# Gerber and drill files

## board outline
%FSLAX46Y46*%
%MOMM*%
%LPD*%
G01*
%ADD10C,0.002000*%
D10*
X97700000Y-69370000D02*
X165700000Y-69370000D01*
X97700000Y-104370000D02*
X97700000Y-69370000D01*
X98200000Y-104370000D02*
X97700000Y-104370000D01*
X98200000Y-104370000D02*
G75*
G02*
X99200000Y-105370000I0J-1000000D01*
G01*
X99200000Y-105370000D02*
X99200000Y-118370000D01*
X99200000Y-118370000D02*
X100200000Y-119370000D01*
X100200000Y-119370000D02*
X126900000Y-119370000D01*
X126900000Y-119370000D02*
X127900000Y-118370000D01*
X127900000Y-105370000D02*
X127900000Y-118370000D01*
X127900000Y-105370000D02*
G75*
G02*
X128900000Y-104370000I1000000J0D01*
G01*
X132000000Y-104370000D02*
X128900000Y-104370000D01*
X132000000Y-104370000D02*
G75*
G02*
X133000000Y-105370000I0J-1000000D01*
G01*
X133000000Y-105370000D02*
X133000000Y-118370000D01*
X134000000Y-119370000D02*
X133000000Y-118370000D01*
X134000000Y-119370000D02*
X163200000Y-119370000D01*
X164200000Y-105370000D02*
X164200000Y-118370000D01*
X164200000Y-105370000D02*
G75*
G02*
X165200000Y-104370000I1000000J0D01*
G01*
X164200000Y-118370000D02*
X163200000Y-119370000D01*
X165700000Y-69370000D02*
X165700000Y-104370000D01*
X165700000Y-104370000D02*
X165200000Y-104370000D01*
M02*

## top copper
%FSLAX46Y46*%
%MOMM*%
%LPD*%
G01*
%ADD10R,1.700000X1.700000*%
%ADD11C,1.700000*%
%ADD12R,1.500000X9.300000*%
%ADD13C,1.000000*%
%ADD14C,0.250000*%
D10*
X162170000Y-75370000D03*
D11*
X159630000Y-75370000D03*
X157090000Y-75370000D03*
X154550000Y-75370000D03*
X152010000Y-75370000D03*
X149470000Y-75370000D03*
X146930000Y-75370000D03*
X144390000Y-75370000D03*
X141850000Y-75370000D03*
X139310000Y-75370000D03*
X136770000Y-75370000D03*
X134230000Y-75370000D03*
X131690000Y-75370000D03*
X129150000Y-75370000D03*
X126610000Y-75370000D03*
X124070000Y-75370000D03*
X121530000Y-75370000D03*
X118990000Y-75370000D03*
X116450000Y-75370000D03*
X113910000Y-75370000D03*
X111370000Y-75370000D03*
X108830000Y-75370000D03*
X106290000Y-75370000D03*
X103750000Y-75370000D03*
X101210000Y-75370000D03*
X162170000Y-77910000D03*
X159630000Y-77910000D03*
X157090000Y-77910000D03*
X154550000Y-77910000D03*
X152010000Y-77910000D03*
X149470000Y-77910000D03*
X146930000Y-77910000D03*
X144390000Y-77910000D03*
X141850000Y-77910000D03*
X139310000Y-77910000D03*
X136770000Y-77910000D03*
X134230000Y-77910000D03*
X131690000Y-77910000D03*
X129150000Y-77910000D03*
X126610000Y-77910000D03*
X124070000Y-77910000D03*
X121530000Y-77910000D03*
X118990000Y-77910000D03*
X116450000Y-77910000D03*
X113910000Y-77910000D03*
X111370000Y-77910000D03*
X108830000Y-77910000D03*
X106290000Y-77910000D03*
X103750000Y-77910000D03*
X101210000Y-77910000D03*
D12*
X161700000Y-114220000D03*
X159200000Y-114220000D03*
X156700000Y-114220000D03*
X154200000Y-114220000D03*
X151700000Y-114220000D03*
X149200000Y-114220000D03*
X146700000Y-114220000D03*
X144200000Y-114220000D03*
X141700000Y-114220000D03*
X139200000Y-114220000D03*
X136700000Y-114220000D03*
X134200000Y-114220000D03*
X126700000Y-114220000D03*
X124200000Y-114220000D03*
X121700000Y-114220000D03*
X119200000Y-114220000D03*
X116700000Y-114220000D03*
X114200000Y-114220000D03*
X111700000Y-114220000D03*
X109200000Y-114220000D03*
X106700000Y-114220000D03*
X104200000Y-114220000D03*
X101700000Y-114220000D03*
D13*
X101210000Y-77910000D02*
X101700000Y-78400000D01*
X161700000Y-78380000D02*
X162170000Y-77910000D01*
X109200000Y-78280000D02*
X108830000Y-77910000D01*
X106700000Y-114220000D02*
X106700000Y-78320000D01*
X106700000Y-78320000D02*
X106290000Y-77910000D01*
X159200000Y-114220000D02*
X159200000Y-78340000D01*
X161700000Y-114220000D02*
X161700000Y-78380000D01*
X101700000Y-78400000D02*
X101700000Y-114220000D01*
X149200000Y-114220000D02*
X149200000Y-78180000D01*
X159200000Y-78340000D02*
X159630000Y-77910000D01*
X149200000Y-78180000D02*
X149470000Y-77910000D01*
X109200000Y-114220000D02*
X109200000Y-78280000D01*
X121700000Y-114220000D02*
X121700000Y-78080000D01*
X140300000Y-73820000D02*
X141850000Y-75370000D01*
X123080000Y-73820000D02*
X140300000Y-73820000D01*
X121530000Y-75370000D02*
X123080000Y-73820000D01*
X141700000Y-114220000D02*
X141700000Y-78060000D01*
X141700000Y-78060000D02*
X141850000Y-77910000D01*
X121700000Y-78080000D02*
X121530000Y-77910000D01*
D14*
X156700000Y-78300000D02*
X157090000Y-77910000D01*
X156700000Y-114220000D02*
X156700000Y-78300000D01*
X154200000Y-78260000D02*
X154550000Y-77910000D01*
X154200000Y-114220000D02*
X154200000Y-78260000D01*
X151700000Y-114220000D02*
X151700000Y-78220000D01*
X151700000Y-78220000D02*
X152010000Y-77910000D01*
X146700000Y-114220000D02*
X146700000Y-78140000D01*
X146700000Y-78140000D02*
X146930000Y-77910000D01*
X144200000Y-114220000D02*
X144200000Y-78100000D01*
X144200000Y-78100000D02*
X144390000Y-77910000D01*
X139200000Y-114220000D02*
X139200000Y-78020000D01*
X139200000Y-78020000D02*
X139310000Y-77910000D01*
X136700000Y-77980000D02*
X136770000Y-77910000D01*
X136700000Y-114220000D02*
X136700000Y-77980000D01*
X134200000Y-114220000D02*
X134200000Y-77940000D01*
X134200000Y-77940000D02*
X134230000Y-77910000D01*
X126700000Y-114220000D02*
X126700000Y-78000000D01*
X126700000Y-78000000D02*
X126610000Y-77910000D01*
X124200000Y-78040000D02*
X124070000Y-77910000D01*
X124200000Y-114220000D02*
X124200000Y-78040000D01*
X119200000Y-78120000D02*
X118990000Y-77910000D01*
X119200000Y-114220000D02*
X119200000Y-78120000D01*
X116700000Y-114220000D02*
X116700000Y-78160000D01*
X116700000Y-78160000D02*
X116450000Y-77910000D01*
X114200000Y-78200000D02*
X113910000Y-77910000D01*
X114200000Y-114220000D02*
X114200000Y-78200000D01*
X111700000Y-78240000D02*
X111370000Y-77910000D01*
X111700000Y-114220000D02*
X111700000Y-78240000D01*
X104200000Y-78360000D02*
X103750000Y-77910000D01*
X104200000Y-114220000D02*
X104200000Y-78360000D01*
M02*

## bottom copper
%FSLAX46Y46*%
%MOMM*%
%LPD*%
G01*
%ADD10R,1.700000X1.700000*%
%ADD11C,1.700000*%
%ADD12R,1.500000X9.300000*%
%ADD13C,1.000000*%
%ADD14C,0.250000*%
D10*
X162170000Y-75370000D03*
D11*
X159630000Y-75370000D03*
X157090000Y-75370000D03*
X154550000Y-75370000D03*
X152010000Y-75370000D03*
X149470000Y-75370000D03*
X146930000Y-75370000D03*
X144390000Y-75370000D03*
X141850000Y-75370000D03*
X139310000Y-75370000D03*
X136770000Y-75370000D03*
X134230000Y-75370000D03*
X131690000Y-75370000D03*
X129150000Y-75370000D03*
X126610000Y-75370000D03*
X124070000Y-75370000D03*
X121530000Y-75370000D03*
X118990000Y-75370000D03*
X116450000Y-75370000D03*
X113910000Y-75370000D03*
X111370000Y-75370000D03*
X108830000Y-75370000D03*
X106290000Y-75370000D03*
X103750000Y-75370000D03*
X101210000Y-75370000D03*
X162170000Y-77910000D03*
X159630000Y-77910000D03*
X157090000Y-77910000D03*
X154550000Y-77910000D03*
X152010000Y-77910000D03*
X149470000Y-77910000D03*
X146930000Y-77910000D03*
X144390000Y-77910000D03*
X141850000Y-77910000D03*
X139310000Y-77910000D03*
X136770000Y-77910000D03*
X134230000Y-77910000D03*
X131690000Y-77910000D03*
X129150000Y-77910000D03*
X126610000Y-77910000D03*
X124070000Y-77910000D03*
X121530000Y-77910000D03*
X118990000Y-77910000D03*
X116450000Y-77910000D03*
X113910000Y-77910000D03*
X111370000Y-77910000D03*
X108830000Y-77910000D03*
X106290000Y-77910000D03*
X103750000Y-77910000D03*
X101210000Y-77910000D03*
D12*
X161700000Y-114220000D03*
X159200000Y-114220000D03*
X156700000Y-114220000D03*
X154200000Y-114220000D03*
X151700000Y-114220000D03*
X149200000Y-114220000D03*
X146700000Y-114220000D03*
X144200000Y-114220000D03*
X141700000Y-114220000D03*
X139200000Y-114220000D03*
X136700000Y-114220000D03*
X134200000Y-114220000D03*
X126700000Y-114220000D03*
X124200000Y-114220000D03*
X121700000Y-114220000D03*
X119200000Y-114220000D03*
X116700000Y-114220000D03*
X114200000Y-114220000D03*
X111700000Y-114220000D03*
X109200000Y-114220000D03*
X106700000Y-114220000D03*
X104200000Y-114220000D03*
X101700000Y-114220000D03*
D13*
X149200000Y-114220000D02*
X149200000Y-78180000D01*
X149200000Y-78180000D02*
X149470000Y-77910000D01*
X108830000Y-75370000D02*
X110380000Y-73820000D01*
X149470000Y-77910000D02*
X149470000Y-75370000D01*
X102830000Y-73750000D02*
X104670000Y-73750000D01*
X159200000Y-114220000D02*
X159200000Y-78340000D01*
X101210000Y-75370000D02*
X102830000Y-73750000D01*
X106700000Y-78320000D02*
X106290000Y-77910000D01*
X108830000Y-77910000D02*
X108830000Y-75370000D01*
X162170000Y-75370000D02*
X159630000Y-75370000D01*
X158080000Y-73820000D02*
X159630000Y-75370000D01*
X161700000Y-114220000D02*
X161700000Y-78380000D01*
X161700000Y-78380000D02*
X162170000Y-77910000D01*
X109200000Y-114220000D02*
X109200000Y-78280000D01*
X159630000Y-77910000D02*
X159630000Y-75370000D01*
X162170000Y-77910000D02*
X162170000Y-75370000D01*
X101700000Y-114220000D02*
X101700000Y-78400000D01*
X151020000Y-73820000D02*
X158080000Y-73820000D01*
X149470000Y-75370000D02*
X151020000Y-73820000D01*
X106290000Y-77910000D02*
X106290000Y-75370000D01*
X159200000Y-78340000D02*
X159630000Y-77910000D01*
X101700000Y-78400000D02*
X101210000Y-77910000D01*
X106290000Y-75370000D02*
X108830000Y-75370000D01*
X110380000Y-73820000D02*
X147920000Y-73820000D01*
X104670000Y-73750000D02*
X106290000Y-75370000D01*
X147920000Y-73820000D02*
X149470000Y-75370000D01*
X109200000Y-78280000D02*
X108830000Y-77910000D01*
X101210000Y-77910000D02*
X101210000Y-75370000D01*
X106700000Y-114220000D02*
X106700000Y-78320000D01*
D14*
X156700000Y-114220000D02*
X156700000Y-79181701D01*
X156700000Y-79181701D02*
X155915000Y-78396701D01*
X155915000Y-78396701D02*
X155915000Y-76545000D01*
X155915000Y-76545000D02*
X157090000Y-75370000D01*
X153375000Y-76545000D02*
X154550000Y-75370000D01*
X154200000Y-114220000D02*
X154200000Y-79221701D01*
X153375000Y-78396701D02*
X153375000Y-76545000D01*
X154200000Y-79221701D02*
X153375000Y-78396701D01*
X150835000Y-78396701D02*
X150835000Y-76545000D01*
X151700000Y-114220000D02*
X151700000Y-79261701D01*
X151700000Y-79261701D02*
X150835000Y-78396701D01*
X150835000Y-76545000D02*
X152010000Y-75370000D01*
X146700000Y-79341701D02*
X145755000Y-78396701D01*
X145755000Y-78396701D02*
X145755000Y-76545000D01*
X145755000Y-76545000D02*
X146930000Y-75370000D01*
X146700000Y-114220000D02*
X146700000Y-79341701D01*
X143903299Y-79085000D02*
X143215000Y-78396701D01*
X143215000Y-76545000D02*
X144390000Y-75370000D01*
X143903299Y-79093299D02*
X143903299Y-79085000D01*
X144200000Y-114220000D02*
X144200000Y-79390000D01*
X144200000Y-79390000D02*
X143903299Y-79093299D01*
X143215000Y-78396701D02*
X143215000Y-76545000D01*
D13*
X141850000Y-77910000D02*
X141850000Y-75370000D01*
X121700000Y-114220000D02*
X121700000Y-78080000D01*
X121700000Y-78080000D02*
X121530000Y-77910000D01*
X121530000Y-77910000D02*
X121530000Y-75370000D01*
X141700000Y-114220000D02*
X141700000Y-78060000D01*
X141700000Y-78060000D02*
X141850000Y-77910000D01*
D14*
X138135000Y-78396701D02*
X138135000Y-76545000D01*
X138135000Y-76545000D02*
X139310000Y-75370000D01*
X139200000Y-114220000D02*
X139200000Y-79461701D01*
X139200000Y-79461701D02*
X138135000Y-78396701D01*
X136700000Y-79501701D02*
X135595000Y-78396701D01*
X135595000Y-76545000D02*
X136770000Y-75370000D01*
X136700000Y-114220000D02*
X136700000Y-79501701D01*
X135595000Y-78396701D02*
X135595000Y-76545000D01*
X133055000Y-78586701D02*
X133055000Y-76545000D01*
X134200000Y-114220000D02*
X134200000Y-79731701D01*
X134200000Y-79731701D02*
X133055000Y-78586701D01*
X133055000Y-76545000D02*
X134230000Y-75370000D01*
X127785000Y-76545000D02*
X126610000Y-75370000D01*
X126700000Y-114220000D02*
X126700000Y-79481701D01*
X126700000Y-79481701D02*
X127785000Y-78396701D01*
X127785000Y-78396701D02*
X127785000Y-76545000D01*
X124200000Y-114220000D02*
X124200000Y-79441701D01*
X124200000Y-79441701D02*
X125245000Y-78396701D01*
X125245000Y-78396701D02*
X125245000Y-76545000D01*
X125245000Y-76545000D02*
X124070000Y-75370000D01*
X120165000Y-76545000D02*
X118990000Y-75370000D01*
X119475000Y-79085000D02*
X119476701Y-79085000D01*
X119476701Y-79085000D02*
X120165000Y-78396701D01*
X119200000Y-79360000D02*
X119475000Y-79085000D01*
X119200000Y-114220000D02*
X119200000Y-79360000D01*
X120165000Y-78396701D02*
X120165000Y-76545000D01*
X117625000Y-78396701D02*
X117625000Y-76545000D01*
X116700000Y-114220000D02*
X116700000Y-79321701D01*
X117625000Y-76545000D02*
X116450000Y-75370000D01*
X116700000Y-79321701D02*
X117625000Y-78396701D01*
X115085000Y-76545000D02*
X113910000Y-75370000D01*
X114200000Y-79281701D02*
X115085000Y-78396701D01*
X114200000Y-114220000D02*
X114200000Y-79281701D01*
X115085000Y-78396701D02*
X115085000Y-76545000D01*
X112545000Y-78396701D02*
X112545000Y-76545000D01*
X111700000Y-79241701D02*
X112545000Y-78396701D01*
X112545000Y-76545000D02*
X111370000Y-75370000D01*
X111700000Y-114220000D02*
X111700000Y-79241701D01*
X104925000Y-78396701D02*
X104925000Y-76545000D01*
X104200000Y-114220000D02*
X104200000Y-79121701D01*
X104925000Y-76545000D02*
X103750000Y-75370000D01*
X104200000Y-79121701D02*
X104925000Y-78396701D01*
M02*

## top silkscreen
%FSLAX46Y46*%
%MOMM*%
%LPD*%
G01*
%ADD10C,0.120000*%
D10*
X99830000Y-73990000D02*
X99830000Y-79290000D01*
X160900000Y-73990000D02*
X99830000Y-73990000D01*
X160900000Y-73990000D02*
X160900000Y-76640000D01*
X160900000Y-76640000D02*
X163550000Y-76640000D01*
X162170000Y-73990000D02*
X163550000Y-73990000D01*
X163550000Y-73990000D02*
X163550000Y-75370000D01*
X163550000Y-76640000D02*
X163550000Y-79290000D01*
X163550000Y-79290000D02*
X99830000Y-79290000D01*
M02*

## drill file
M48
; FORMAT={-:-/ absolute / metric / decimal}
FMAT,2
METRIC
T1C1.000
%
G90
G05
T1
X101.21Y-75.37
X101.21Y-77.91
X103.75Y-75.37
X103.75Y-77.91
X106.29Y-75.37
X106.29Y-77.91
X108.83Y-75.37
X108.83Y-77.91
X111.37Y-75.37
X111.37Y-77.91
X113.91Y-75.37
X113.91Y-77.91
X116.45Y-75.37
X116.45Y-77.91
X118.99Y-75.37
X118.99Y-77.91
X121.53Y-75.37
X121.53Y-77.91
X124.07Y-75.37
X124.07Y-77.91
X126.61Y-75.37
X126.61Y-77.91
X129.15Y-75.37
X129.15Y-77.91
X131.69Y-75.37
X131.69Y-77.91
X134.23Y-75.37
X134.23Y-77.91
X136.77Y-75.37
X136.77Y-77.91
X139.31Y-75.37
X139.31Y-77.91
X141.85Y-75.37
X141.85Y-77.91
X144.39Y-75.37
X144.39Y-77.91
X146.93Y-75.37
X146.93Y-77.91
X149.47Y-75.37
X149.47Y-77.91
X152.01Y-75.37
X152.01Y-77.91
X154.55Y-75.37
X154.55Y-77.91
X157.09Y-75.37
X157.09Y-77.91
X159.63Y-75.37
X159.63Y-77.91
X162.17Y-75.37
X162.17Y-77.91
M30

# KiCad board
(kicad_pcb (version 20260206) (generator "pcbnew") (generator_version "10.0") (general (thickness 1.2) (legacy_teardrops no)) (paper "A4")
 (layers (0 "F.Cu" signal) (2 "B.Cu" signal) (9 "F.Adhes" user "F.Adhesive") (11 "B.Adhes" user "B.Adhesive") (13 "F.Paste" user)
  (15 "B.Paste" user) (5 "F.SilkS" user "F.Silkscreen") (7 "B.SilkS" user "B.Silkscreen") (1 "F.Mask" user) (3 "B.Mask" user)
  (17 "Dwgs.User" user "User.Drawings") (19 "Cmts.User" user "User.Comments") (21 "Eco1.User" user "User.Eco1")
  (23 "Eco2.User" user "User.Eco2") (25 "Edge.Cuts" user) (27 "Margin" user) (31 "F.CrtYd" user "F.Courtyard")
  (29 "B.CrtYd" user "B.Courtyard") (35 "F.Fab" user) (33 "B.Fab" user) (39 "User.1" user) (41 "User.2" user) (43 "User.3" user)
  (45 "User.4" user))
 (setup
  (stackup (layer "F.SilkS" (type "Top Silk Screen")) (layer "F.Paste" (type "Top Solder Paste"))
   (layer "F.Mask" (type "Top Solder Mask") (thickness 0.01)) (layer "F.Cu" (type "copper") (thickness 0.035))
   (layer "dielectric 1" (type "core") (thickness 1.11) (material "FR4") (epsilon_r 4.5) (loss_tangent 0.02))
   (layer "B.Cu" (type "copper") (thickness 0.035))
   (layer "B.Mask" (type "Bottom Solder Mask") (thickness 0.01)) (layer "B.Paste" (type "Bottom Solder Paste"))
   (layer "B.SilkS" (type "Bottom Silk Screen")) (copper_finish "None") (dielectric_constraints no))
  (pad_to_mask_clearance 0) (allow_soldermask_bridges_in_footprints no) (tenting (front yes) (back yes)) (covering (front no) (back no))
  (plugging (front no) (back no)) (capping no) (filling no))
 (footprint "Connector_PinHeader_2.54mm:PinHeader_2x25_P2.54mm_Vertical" (layer "F.Cu") (at 162.17 75.37 -90)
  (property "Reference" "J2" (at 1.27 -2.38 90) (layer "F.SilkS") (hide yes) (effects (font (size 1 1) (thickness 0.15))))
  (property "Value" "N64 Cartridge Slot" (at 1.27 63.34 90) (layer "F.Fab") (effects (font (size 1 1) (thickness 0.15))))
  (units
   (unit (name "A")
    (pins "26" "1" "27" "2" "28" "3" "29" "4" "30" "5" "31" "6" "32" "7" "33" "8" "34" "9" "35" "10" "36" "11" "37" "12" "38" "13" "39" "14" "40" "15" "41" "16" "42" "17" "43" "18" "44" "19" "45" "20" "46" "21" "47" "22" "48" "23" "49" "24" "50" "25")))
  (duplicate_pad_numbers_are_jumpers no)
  (fp_line (start -1.38 62.34) (end 3.92 62.34) (stroke (width 0.12) (type solid)) (layer "F.SilkS"))
  (fp_line (start -1.38 1.27) (end -1.38 62.34) (stroke (width 0.12) (type solid)) (layer "F.SilkS"))
  (fp_line (start -1.38 1.27) (end 1.27 1.27) (stroke (width 0.12) (type solid)) (layer "F.SilkS"))
  (fp_line (start 1.27 1.27) (end 1.27 -1.38) (stroke (width 0.12) (type solid)) (layer "F.SilkS"))
  (fp_line (start -1.38 0) (end -1.38 -1.38) (stroke (width 0.12) (type solid)) (layer "F.SilkS"))
  (fp_line (start -1.38 -1.38) (end 0 -1.38) (stroke (width 0.12) (type solid)) (layer "F.SilkS"))
  (fp_line (start 1.27 -1.38) (end 3.92 -1.38) (stroke (width 0.12) (type solid)) (layer "F.SilkS"))
  (fp_line (start 3.92 -1.38) (end 3.92 62.34) (stroke (width 0.12) (type solid)) (layer "F.SilkS"))
  (pad "1" thru_hole rect (at 0 0 270) (size 1.7 1.7) (drill 1) (layers "*.Cu" "*.Mask") (remove_unused_layers no) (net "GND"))
  (pad "2" thru_hole circle (at 0 2.54 270) (size 1.7 1.7) (drill 1) (layers "*.Cu" "*.Mask") (remove_unused_layers no) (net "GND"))
  (pad "3" thru_hole circle (at 0 5.08 270) (size 1.7 1.7) (drill 1) (layers "*.Cu" "*.Mask") (remove_unused_layers no) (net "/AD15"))
  (pad "4" thru_hole circle (at 0 7.62 270) (size 1.7 1.7) (drill 1) (layers "*.Cu" "*.Mask") (remove_unused_layers no) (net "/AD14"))
  (pad "5" thru_hole circle (at 0 10.16 270) (size 1.7 1.7) (drill 1) (layers "*.Cu" "*.Mask") (remove_unused_layers no) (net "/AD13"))
  (pad "6" thru_hole circle (at 0 12.7 270) (size 1.7 1.7) (drill 1) (layers "*.Cu" "*.Mask") (remove_unused_layers no) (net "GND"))
  (pad "7" thru_hole circle (at 0 15.24 270) (size 1.7 1.7) (drill 1) (layers "*.Cu" "*.Mask") (remove_unused_layers no) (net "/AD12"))
  (pad "8" thru_hole circle (at 0 17.78 270) (size 1.7 1.7) (drill 1) (layers "*.Cu" "*.Mask") (remove_unused_layers no) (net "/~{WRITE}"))
  (pad "9" thru_hole circle (at 0 20.32 270) (size 1.7 1.7) (drill 1) (layers "*.Cu" "*.Mask") (remove_unused_layers no) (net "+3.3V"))
  (pad "10" thru_hole circle (at 0 22.86 270) (size 1.7 1.7) (drill 1) (layers "*.Cu" "*.Mask") (remove_unused_layers no) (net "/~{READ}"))
  (pad "11" thru_hole circle (at 0 25.4 270) (size 1.7 1.7) (drill 1) (layers "*.Cu" "*.Mask") (remove_unused_layers no) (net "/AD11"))
  (pad "12" thru_hole circle (at 0 27.94 270) (size 1.7 1.7) (drill 1) (layers "*.Cu" "*.Mask") (remove_unused_layers no) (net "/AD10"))
  (pad "13" thru_hole circle (at 0 30.48 270) (size 1.7 1.7) (drill 1) (layers "*.Cu" "*.Mask") (remove_unused_layers no)
   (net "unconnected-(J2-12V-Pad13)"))
  (pad "14" thru_hole circle (at 0 33.02 270) (size 1.7 1.7) (drill 1) (layers "*.Cu" "*.Mask") (remove_unused_layers no)
   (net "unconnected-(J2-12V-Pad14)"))
  (pad "15" thru_hole circle (at 0 35.56 270) (size 1.7 1.7) (drill 1) (layers "*.Cu" "*.Mask") (remove_unused_layers no) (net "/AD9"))
  (pad "16" thru_hole circle (at 0 38.1 270) (size 1.7 1.7) (drill 1) (layers "*.Cu" "*.Mask") (remove_unused_layers no) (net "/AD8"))
  (pad "17" thru_hole circle (at 0 40.64 270) (size 1.7 1.7) (drill 1) (layers "*.Cu" "*.Mask") (remove_unused_layers no) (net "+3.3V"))
  (pad "18" thru_hole circle (at 0 43.18 270) (size 1.7 1.7) (drill 1) (layers "*.Cu" "*.Mask") (remove_unused_layers no) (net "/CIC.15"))
  (pad "19" thru_hole circle (at 0 45.72 270) (size 1.7 1.7) (drill 1) (layers "*.Cu" "*.Mask") (remove_unused_layers no) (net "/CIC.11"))
  (pad "20" thru_hole circle (at 0 48.26 270) (size 1.7 1.7) (drill 1) (layers "*.Cu" "*.Mask") (remove_unused_layers no)
   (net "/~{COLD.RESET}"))
  (pad "21" thru_hole circle (at 0 50.8 270) (size 1.7 1.7) (drill 1) (layers "*.Cu" "*.Mask") (remove_unused_layers no) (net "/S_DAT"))
  (pad "22" thru_hole circle (at 0 53.34 270) (size 1.7 1.7) (drill 1) (layers "*.Cu" "*.Mask") (remove_unused_layers no) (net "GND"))
  (pad "23" thru_hole circle (at 0 55.88 270) (size 1.7 1.7) (drill 1) (layers "*.Cu" "*.Mask") (remove_unused_layers no) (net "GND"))
  (pad "24" thru_hole circle (at 0 58.42 270) (size 1.7 1.7) (drill 1) (layers "*.Cu" "*.Mask") (remove_unused_layers no) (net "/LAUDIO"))
  (pad "25" thru_hole circle (at 0 60.96 270) (size 1.7 1.7) (drill 1) (layers "*.Cu" "*.Mask") (remove_unused_layers no) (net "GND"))
  (pad "26" thru_hole circle (at 2.54 0 270) (size 1.7 1.7) (drill 1) (layers "*.Cu" "*.Mask") (remove_unused_layers no) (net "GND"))
  (pad "27" thru_hole circle (at 2.54 2.54 270) (size 1.7 1.7) (drill 1) (layers "*.Cu" "*.Mask") (remove_unused_layers no) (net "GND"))
  (pad "28" thru_hole circle (at 2.54 5.08 270) (size 1.7 1.7) (drill 1) (layers "*.Cu" "*.Mask") (remove_unused_layers no) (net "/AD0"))
  (pad "29" thru_hole circle (at 2.54 7.62 270) (size 1.7 1.7) (drill 1) (layers "*.Cu" "*.Mask") (remove_unused_layers no) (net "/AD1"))
  (pad "30" thru_hole circle (at 2.54 10.16 270) (size 1.7 1.7) (drill 1) (layers "*.Cu" "*.Mask") (remove_unused_layers no) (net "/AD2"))
  (pad "31" thru_hole circle (at 2.54 12.7 270) (size 1.7 1.7) (drill 1) (layers "*.Cu" "*.Mask") (remove_unused_layers no) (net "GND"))
  (pad "32" thru_hole circle (at 2.54 15.24 270) (size 1.7 1.7) (drill 1) (layers "*.Cu" "*.Mask") (remove_unused_layers no) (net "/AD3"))
  (pad "33" thru_hole circle (at 2.54 17.78 270) (size 1.7 1.7) (drill 1) (layers "*.Cu" "*.Mask") (remove_unused_layers no) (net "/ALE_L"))
  (pad "34" thru_hole circle (at 2.54 20.32 270) (size 1.7 1.7) (drill 1) (layers "*.Cu" "*.Mask") (remove_unused_layers no) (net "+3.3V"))
  (pad "35" thru_hole circle (at 2.54 22.86 270) (size 1.7 1.7) (drill 1) (layers "*.Cu" "*.Mask") (remove_unused_layers no) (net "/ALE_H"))
  (pad "36" thru_hole circle (at 2.54 25.4 270) (size 1.7 1.7) (drill 1) (layers "*.Cu" "*.Mask") (remove_unused_layers no) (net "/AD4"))
  (pad "37" thru_hole circle (at 2.54 27.94 270) (size 1.7 1.7) (drill 1) (layers "*.Cu" "*.Mask") (remove_unused_layers no) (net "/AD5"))
  (pad "38" thru_hole circle (at 2.54 30.48 270) (size 1.7 1.7) (drill 1) (layers "*.Cu" "*.Mask") (remove_unused_layers no)
   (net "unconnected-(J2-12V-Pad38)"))
  (pad "39" thru_hole circle (at 2.54 33.02 270) (size 1.7 1.7) (drill 1) (layers "*.Cu" "*.Mask") (remove_unused_layers no)
   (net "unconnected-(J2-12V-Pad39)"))
  (pad "40" thru_hole circle (at 2.54 35.56 270) (size 1.7 1.7) (drill 1) (layers "*.Cu" "*.Mask") (remove_unused_layers no) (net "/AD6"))
  (pad "41" thru_hole circle (at 2.54 38.1 270) (size 1.7 1.7) (drill 1) (layers "*.Cu" "*.Mask") (remove_unused_layers no) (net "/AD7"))
  (pad "42" thru_hole circle (at 2.54 40.64 270) (size 1.7 1.7) (drill 1) (layers "*.Cu" "*.Mask") (remove_unused_layers no) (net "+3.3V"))
  (pad "43" thru_hole circle (at 2.54 43.18 270) (size 1.7 1.7) (drill 1) (layers "*.Cu" "*.Mask") (remove_unused_layers no) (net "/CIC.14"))
  (pad "44" thru_hole circle (at 2.54 45.72 270) (size 1.7 1.7) (drill 1) (layers "*.Cu" "*.Mask") (remove_unused_layers no)
   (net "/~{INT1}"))
  (pad "45" thru_hole circle (at 2.54 48.26 270) (size 1.7 1.7) (drill 1) (layers "*.Cu" "*.Mask") (remove_unused_layers no) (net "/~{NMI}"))
  (pad "46" thru_hole circle (at 2.54 50.8 270) (size 1.7 1.7) (drill 1) (layers "*.Cu" "*.Mask") (remove_unused_layers no)
   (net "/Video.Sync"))
  (pad "47" thru_hole circle (at 2.54 53.34 270) (size 1.7 1.7) (drill 1) (layers "*.Cu" "*.Mask") (remove_unused_layers no) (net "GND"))
  (pad "48" thru_hole circle (at 2.54 55.88 270) (size 1.7 1.7) (drill 1) (layers "*.Cu" "*.Mask") (remove_unused_layers no) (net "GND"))
  (pad "49" thru_hole circle (at 2.54 58.42 270) (size 1.7 1.7) (drill 1) (layers "*.Cu" "*.Mask") (remove_unused_layers no) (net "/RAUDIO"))
  (pad "50" thru_hole circle (at 2.54 60.96 270) (size 1.7 1.7) (drill 1) (layers "*.Cu" "*.Mask") (remove_unused_layers no) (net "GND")))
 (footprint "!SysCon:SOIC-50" (layer "B.Cu") (at 131.7 114.22)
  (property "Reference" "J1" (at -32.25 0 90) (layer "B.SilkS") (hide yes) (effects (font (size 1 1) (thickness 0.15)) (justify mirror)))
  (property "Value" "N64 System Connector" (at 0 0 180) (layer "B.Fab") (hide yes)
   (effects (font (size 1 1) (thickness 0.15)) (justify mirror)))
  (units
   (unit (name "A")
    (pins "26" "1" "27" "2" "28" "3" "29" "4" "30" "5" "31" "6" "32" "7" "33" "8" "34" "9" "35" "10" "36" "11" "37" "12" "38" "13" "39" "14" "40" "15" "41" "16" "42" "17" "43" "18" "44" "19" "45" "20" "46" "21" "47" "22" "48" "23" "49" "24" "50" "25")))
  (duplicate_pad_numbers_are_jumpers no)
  (pad "1" smd rect (at 30 0) (size 1.5 9.3) (layers "B.Cu" "B.Mask" "B.Paste") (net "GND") (thermal_bridge_angle 45))
  (pad "2" smd rect (at 27.5 0) (size 1.5 9.3) (layers "B.Cu" "B.Mask" "B.Paste") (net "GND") (thermal_bridge_angle 45))
  (pad "3" smd rect (at 25 0) (size 1.5 9.3) (layers "B.Cu" "B.Mask" "B.Paste") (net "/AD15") (thermal_bridge_angle 45))
  (pad "4" smd rect (at 22.5 0) (size 1.5 9.3) (layers "B.Cu" "B.Mask" "B.Paste") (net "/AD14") (thermal_bridge_angle 45))
  (pad "5" smd rect (at 20 0) (size 1.5 9.3) (layers "B.Cu" "B.Mask" "B.Paste") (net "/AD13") (thermal_bridge_angle 45))
  (pad "6" smd rect (at 17.5 0) (size 1.5 9.3) (layers "B.Cu" "B.Mask" "B.Paste") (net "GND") (thermal_bridge_angle 45))
  (pad "7" smd rect (at 15 0) (size 1.5 9.3) (layers "B.Cu" "B.Mask" "B.Paste") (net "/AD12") (thermal_bridge_angle 45))
  (pad "8" smd rect (at 12.5 0) (size 1.5 9.3) (layers "B.Cu" "B.Mask" "B.Paste") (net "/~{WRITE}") (thermal_bridge_angle 45))
  (pad "9" smd rect (at 10 0) (size 1.5 9.3) (layers "B.Cu" "B.Mask" "B.Paste") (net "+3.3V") (thermal_bridge_angle 45))
  (pad "10" smd rect (at 7.5 0) (size 1.5 9.3) (layers "B.Cu" "B.Mask" "B.Paste") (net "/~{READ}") (thermal_bridge_angle 45))
  (pad "11" smd rect (at 5 0) (size 1.5 9.3) (layers "B.Cu" "B.Mask" "B.Paste") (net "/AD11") (thermal_bridge_angle 45))
  (pad "12" smd rect (at 2.5 0) (size 1.5 9.3) (layers "B.Cu" "B.Mask" "B.Paste") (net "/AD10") (thermal_bridge_angle 45))
  (pad "15" smd rect (at -5 0) (size 1.5 9.3) (layers "B.Cu" "B.Mask" "B.Paste") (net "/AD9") (thermal_bridge_angle 45))
  (pad "16" smd rect (at -7.5 0) (size 1.5 9.3) (layers "B.Cu" "B.Mask" "B.Paste") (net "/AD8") (thermal_bridge_angle 45))
  (pad "17" smd rect (at -10 0) (size 1.5 9.3) (layers "B.Cu" "B.Mask" "B.Paste") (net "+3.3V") (thermal_bridge_angle 45))
  (pad "18" smd rect (at -12.5 0) (size 1.5 9.3) (layers "B.Cu" "B.Mask" "B.Paste") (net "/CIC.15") (thermal_bridge_angle 45))
  (pad "19" smd rect (at -15 0) (size 1.5 9.3) (layers "B.Cu" "B.Mask" "B.Paste") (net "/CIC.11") (thermal_bridge_angle 45))
  (pad "20" smd rect (at -17.5 0) (size 1.5 9.3) (layers "B.Cu" "B.Mask" "B.Paste") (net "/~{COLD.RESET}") (thermal_bridge_angle 45))
  (pad "21" smd rect (at -20 0) (size 1.5 9.3) (layers "B.Cu" "B.Mask" "B.Paste") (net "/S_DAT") (thermal_bridge_angle 45))
  (pad "22" smd rect (at -22.5 0) (size 1.5 9.3) (layers "B.Cu" "B.Mask" "B.Paste") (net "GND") (thermal_bridge_angle 45))
  (pad "23" smd rect (at -25 0) (size 1.5 9.3) (layers "B.Cu" "B.Mask" "B.Paste") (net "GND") (thermal_bridge_angle 45))
  (pad "24" smd rect (at -27.5 0) (size 1.5 9.3) (layers "B.Cu" "B.Mask" "B.Paste") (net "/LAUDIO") (thermal_bridge_angle 45))
  (pad "25" smd rect (at -30 0) (size 1.5 9.3) (layers "B.Cu" "B.Mask" "B.Paste") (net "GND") (thermal_bridge_angle 45))
  (pad "26" smd rect (at 30 0) (size 1.5 9.3) (layers "F.Cu" "F.Mask") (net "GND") (thermal_bridge_angle 45))
  (pad "27" smd rect (at 27.5 0) (size 1.5 9.3) (layers "F.Cu" "F.Mask") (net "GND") (thermal_bridge_angle 45))
  (pad "28" smd rect (at 25 0) (size 1.5 9.3) (layers "F.Cu" "F.Mask") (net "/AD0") (thermal_bridge_angle 45))
  (pad "29" smd rect (at 22.5 0) (size 1.5 9.3) (layers "F.Cu" "F.Mask") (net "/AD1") (thermal_bridge_angle 45))
  (pad "30" smd rect (at 20 0) (size 1.5 9.3) (layers "F.Cu" "F.Mask") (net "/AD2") (thermal_bridge_angle 45))
  (pad "31" smd rect (at 17.5 0) (size 1.5 9.3) (layers "F.Cu" "F.Mask") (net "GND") (thermal_bridge_angle 45))
  (pad "32" smd rect (at 15 0) (size 1.5 9.3) (layers "F.Cu" "F.Mask") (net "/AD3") (thermal_bridge_angle 45))
  (pad "33" smd rect (at 12.5 0) (size 1.5 9.3) (layers "F.Cu" "F.Mask") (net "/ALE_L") (thermal_bridge_angle 45))
  (pad "34" smd rect (at 10 0) (size 1.5 9.3) (layers "F.Cu" "F.Mask") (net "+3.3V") (thermal_bridge_angle 45))
  (pad "35" smd rect (at 7.5 0) (size 1.5 9.3) (layers "F.Cu" "F.Mask") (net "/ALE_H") (thermal_bridge_angle 45))
  (pad "36" smd rect (at 5 0) (size 1.5 9.3) (layers "F.Cu" "F.Mask") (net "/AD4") (thermal_bridge_angle 45))
  (pad "37" smd rect (at 2.5 0) (size 1.5 9.3) (layers "F.Cu" "F.Mask") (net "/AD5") (thermal_bridge_angle 45))
  (pad "40" smd rect (at -5 0) (size 1.5 9.3) (layers "F.Cu" "F.Mask") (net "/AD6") (thermal_bridge_angle 45))
  (pad "41" smd rect (at -7.5 0) (size 1.5 9.3) (layers "F.Cu" "F.Mask") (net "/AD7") (thermal_bridge_angle 45))
  (pad "42" smd rect (at -10 0) (size 1.5 9.3) (layers "F.Cu" "F.Mask") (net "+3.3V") (thermal_bridge_angle 45))
  (pad "43" smd rect (at -12.5 0) (size 1.5 9.3) (layers "F.Cu" "F.Mask") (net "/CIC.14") (thermal_bridge_angle 45))
  (pad "44" smd rect (at -15 0) (size 1.5 9.3) (layers "F.Cu" "F.Mask") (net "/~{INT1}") (thermal_bridge_angle 45))
  (pad "45" smd rect (at -17.5 0) (size 1.5 9.3) (layers "F.Cu" "F.Mask") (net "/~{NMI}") (thermal_bridge_angle 45))
  (pad "46" smd rect (at -20 0) (size 1.5 9.3) (layers "F.Cu" "F.Mask") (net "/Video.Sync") (thermal_bridge_angle 45))
  (pad "47" smd rect (at -22.5 0) (size 1.5 9.3) (layers "F.Cu" "F.Mask") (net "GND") (thermal_bridge_angle 45))
  (pad "48" smd rect (at -25 0) (size 1.5 9.3) (layers "F.Cu" "F.Mask") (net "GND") (thermal_bridge_angle 45))
  (pad "49" smd rect (at -27.5 0) (size 1.5 9.3) (layers "F.Cu" "F.Mask") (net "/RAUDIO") (thermal_bridge_angle 45))
  (pad "50" smd rect (at -30 0) (size 1.5 9.3) (layers "F.Cu" "F.Mask") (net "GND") (thermal_bridge_angle 45)))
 (gr_line (start 97.7 69.37) (end 165.7 69.37) (stroke (width 0.002) (type solid)) (layer "Edge.Cuts"))
 (gr_line (start 97.7 104.37) (end 97.7 69.37) (stroke (width 0.002) (type solid)) (layer "Edge.Cuts"))
 (gr_line (start 98.2 104.37) (end 97.7 104.37) (stroke (width 0.002) (type solid)) (layer "Edge.Cuts"))
 (gr_arc (start 98.2 104.37) (mid 98.907107 104.662893) (end 99.2 105.37) (stroke (width 0.002) (type default)) (layer "Edge.Cuts"))
 (gr_line (start 99.2 105.37) (end 99.2 118.37) (stroke (width 0.002) (type solid)) (layer "Edge.Cuts"))
 (gr_line (start 99.2 118.37) (end 100.2 119.37) (stroke (width 0.002) (type default)) (layer "Edge.Cuts"))
 (gr_line (start 100.2 119.37) (end 126.9 119.37) (stroke (width 0.002) (type solid)) (layer "Edge.Cuts"))
 (gr_line (start 126.9 119.37) (end 127.9 118.37) (stroke (width 0.002) (type default)) (layer "Edge.Cuts"))
 (gr_line (start 127.9 105.37) (end 127.9 118.37) (stroke (width 0.002) (type solid)) (layer "Edge.Cuts"))
 (gr_arc (start 127.9 105.37) (mid 128.192893 104.662893) (end 128.9 104.37) (stroke (width 0.002) (type default)) (layer "Edge.Cuts"))
 (gr_line (start 132 104.37) (end 128.9 104.37) (stroke (width 0.002) (type solid)) (layer "Edge.Cuts"))
 (gr_arc (start 132 104.37) (mid 132.707107 104.662893) (end 133 105.37) (stroke (width 0.002) (type default)) (layer "Edge.Cuts"))
 (gr_line (start 133 105.37) (end 133 118.37) (stroke (width 0.002) (type solid)) (layer "Edge.Cuts"))
 (gr_line (start 134 119.37) (end 133 118.37) (stroke (width 0.002) (type default)) (layer "Edge.Cuts"))
 (gr_line (start 134 119.37) (end 163.2 119.37) (stroke (width 0.002) (type solid)) (layer "Edge.Cuts"))
 (gr_line (start 164.2 105.37) (end 164.2 118.37) (stroke (width 0.002) (type solid)) (layer "Edge.Cuts"))
 (gr_arc (start 164.2 105.37) (mid 164.492893 104.662893) (end 165.2 104.37) (stroke (width 0.002) (type default)) (layer "Edge.Cuts"))
 (gr_line (start 164.2 118.37) (end 163.2 119.37) (stroke (width 0.002) (type default)) (layer "Edge.Cuts"))
 (gr_line (start 165.7 69.37) (end 165.7 104.37) (stroke (width 0.002) (type solid)) (layer "Edge.Cuts"))
 (gr_line (start 165.7 104.37) (end 165.2 104.37) (stroke (width 0.002) (type solid)) (layer "Edge.Cuts"))
 (segment (start 101.21 77.91) (end 101.7 78.4) (width 1) (layer "F.Cu") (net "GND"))
 (segment (start 161.7 78.38) (end 162.17 77.91) (width 1) (layer "F.Cu") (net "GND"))
 (segment (start 109.2 78.28) (end 108.83 77.91) (width 1) (layer "F.Cu") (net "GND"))
 (segment (start 106.7 114.22) (end 106.7 78.32) (width 1) (layer "F.Cu") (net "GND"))
 (segment (start 106.7 78.32) (end 106.29 77.91) (width 1) (layer "F.Cu") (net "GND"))
 (segment (start 159.2 114.22) (end 159.2 78.34) (width 1) (layer "F.Cu") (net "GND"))
 (segment (start 161.7 114.22) (end 161.7 78.38) (width 1) (layer "F.Cu") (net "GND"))
 (segment (start 101.7 78.4) (end 101.7 114.22) (width 1) (layer "F.Cu") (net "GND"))
 (segment (start 149.2 114.22) (end 149.2 78.18) (width 1) (layer "F.Cu") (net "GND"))
 (segment (start 159.2 78.34) (end 159.63 77.91) (width 1) (layer "F.Cu") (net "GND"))
 (segment (start 149.2 78.18) (end 149.47 77.91) (width 1) (layer "F.Cu") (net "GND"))
 (segment (start 109.2 114.22) (end 109.2 78.28) (width 1) (layer "F.Cu") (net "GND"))
 (segment (start 149.2 114.22) (end 149.2 78.18) (width 1) (layer "B.Cu") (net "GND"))
 (segment (start 149.2 78.18) (end 149.47 77.91) (width 1) (layer "B.Cu") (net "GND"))
 (segment (start 108.83 75.37) (end 110.38 73.82) (width 1) (layer "B.Cu") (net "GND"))
 (segment (start 149.47 77.91) (end 149.47 75.37) (width 1) (layer "B.Cu") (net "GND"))
 (segment (start 102.83 73.75) (end 104.67 73.75) (width 1) (layer "B.Cu") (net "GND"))
 (segment (start 159.2 114.22) (end 159.2 78.34) (width 1) (layer "B.Cu") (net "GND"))
 (segment (start 101.21 75.37) (end 102.83 73.75) (width 1) (layer "B.Cu") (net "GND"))
 (segment (start 106.7 78.32) (end 106.29 77.91) (width 1) (layer "B.Cu") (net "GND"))
 (segment (start 108.83 77.91) (end 108.83 75.37) (width 1) (layer "B.Cu") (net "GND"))
 (segment (start 162.17 75.37) (end 159.63 75.37) (width 1) (layer "B.Cu") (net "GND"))
 (segment (start 158.08 73.82) (end 159.63 75.37) (width 1) (layer "B.Cu") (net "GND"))
 (segment (start 161.7 114.22) (end 161.7 78.38) (width 1) (layer "B.Cu") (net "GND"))
 (segment (start 161.7 78.38) (end 162.17 77.91) (width 1) (layer "B.Cu") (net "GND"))
 (segment (start 109.2 114.22) (end 109.2 78.28) (width 1) (layer "B.Cu") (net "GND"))
 (segment (start 159.63 77.91) (end 159.63 75.37) (width 1) (layer "B.Cu") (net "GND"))
 (segment (start 162.17 77.91) (end 162.17 75.37) (width 1) (layer "B.Cu") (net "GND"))
 (segment (start 101.7 114.22) (end 101.7 78.4) (width 1) (layer "B.Cu") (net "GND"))
 (segment (start 151.02 73.82) (end 158.08 73.82) (width 1) (layer "B.Cu") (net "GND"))
 (segment (start 149.47 75.37) (end 151.02 73.82) (width 1) (layer "B.Cu") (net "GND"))
 (segment (start 106.29 77.91) (end 106.29 75.37) (width 1) (layer "B.Cu") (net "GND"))
 (segment (start 159.2 78.34) (end 159.63 77.91) (width 1) (layer "B.Cu") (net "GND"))
 (segment (start 101.7 78.4) (end 101.21 77.91) (width 1) (layer "B.Cu") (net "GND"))
 (segment (start 106.29 75.37) (end 108.83 75.37) (width 1) (layer "B.Cu") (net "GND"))
 (segment (start 110.38 73.82) (end 147.92 73.82) (width 1) (layer "B.Cu") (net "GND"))
 (segment (start 104.67 73.75) (end 106.29 75.37) (width 1) (layer "B.Cu") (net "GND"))
 (segment (start 147.92 73.82) (end 149.47 75.37) (width 1) (layer "B.Cu") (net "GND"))
 (segment (start 109.2 78.28) (end 108.83 77.91) (width 1) (layer "B.Cu") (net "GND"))
 (segment (start 101.21 77.91) (end 101.21 75.37) (width 1) (layer "B.Cu") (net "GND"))
 (segment (start 106.7 114.22) (end 106.7 78.32) (width 1) (layer "B.Cu") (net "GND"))
 (segment (start 156.7 114.22) (end 156.7 79.181701) (width 0.25) (layer "B.Cu") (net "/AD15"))
 (segment (start 156.7 79.181701) (end 155.915 78.396701) (width 0.25) (layer "B.Cu") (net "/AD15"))
 (segment (start 155.915 78.396701) (end 155.915 76.545) (width 0.25) (layer "B.Cu") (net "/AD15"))
 (segment (start 155.915 76.545) (end 157.09 75.37) (width 0.25) (layer "B.Cu") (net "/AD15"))
 (segment (start 153.375 76.545) (end 154.55 75.37) (width 0.25) (layer "B.Cu") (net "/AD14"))
 (segment (start 154.2 114.22) (end 154.2 79.221701) (width 0.25) (layer "B.Cu") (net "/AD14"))
 (segment (start 153.375 78.396701) (end 153.375 76.545) (width 0.25) (layer "B.Cu") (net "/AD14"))
 (segment (start 154.2 79.221701) (end 153.375 78.396701) (width 0.25) (layer "B.Cu") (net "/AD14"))
 (segment (start 150.835 78.396701) (end 150.835 76.545) (width 0.25) (layer "B.Cu") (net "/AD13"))
 (segment (start 151.7 114.22) (end 151.7 79.261701) (width 0.25) (layer "B.Cu") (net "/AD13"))
 (segment (start 151.7 79.261701) (end 150.835 78.396701) (width 0.25) (layer "B.Cu") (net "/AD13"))
 (segment (start 150.835 76.545) (end 152.01 75.37) (width 0.25) (layer "B.Cu") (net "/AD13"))
 (segment (start 146.7 79.341701) (end 145.755 78.396701) (width 0.25) (layer "B.Cu") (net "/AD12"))
 (segment (start 145.755 78.396701) (end 145.755 76.545) (width 0.25) (layer "B.Cu") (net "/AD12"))
 (segment (start 145.755 76.545) (end 146.93 75.37) (width 0.25) (layer "B.Cu") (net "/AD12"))
 (segment (start 146.7 114.22) (end 146.7 79.341701) (width 0.25) (layer "B.Cu") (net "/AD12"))
 (segment (start 143.903299 79.085) (end 143.215 78.396701) (width 0.25) (layer "B.Cu") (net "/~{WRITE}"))
 (segment (start 143.215 76.545) (end 144.39 75.37) (width 0.25) (layer "B.Cu") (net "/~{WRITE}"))
 (segment (start 143.903299 79.093299) (end 143.903299 79.085) (width 0.25) (layer "B.Cu") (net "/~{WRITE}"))
 (segment (start 144.2 114.22) (end 144.2 79.39) (width 0.25) (layer "B.Cu") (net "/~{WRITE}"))
 (segment (start 144.2 79.39) (end 143.903299 79.093299) (width 0.25) (layer "B.Cu") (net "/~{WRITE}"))
 (segment (start 143.215 78.396701) (end 143.215 76.545) (width 0.25) (layer "B.Cu") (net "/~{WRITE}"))
 (segment (start 121.7 114.22) (end 121.7 78.08) (width 1) (layer "F.Cu") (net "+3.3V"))
 (segment (start 140.3 73.82) (end 141.85 75.37) (width 1) (layer "F.Cu") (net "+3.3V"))
 (segment (start 123.08 73.82) (end 140.3 73.82) (width 1) (layer "F.Cu") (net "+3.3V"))
 (segment (start 121.53 75.37) (end 123.08 73.82) (width 1) (layer "F.Cu") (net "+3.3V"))
 (segment (start 141.7 114.22) (end 141.7 78.06) (width 1) (layer "F.Cu") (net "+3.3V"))
 (segment (start 141.7 78.06) (end 141.85 77.91) (width 1) (layer "F.Cu") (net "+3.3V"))
 (segment (start 121.7 78.08) (end 121.53 77.91) (width 1) (layer "F.Cu") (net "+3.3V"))
 (segment (start 141.85 77.91) (end 141.85 75.37) (width 1) (layer "B.Cu") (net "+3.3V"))
 (segment (start 121.7 114.22) (end 121.7 78.08) (width 1) (layer "B.Cu") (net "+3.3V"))
 (segment (start 121.7 78.08) (end 121.53 77.91) (width 1) (layer "B.Cu") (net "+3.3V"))
 (segment (start 121.53 77.91) (end 121.53 75.37) (width 1) (layer "B.Cu") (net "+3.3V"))
 (segment (start 141.7 114.22) (end 141.7 78.06) (width 1) (layer "B.Cu") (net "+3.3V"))
 (segment (start 141.7 78.06) (end 141.85 77.91) (width 1) (layer "B.Cu") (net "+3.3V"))
 (segment (start 138.135 78.396701) (end 138.135 76.545) (width 0.25) (layer "B.Cu") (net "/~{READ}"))
 (segment (start 138.135 76.545) (end 139.31 75.37) (width 0.25) (layer "B.Cu") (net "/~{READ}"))
 (segment (start 139.2 114.22) (end 139.2 79.461701) (width 0.25) (layer "B.Cu") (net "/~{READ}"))
 (segment (start 139.2 79.461701) (end 138.135 78.396701) (width 0.25) (layer "B.Cu") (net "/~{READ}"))
 (segment (start 136.7 79.501701) (end 135.595 78.396701) (width 0.25) (layer "B.Cu") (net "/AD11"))
 (segment (start 135.595 76.545) (end 136.77 75.37) (width 0.25) (layer "B.Cu") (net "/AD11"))
 (segment (start 136.7 114.22) (end 136.7 79.501701) (width 0.25) (layer "B.Cu") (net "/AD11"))
 (segment (start 135.595 78.396701) (end 135.595 76.545) (width 0.25) (layer "B.Cu") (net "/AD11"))
 (segment (start 133.055 78.586701) (end 133.055 76.545) (width 0.25) (layer "B.Cu") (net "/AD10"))
 (segment (start 134.2 114.22) (end 134.2 79.731701) (width 0.25) (layer "B.Cu") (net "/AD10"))
 (segment (start 134.2 79.731701) (end 133.055 78.586701) (width 0.25) (layer "B.Cu") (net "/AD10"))
 (segment (start 133.055 76.545) (end 134.23 75.37) (width 0.25) (layer "B.Cu") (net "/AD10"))
 (segment (start 127.785 76.545) (end 126.61 75.37) (width 0.25) (layer "B.Cu") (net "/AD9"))
 (segment (start 126.7 114.22) (end 126.7 79.481701) (width 0.25) (layer "B.Cu") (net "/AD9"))
 (segment (start 126.7 79.481701) (end 127.785 78.396701) (width 0.25) (layer "B.Cu") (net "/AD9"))
 (segment (start 127.785 78.396701) (end 127.785 76.545) (width 0.25) (layer "B.Cu") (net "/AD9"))
 (segment (start 124.2 114.22) (end 124.2 79.441701) (width 0.25) (layer "B.Cu") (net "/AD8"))
 (segment (start 124.2 79.441701) (end 125.245 78.396701) (width 0.25) (layer "B.Cu") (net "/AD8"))
 (segment (start 125.245 78.396701) (end 125.245 76.545) (width 0.25) (layer "B.Cu") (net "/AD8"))
 (segment (start 125.245 76.545) (end 124.07 75.37) (width 0.25) (layer "B.Cu") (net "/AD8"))
 (segment (start 120.165 76.545) (end 118.99 75.37) (width 0.25) (layer "B.Cu") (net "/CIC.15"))
 (segment (start 119.475 79.085) (end 119.476701 79.085) (width 0.25) (layer "B.Cu") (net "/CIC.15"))
 (segment (start 119.476701 79.085) (end 120.165 78.396701) (width 0.25) (layer "B.Cu") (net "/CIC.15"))
 (segment (start 119.2 79.36) (end 119.475 79.085) (width 0.25) (layer "B.Cu") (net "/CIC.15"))
 (segment (start 119.2 114.22) (end 119.2 79.36) (width 0.25) (layer "B.Cu") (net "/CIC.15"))
 (segment (start 120.165 78.396701) (end 120.165 76.545) (width 0.25) (layer "B.Cu") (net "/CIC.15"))
 (segment (start 117.625 78.396701) (end 117.625 76.545) (width 0.25) (layer "B.Cu") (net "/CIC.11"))
 (segment (start 116.7 114.22) (end 116.7 79.321701) (width 0.25) (layer "B.Cu") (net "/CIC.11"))
 (segment (start 117.625 76.545) (end 116.45 75.37) (width 0.25) (layer "B.Cu") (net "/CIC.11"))
 (segment (start 116.7 79.321701) (end 117.625 78.396701) (width 0.25) (layer "B.Cu") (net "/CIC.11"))
 (segment (start 115.085 76.545) (end 113.91 75.37) (width 0.25) (layer "B.Cu") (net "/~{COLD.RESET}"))
 (segment (start 114.2 79.281701) (end 115.085 78.396701) (width 0.25) (layer "B.Cu") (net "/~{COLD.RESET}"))
 (segment (start 114.2 114.22) (end 114.2 79.281701) (width 0.25) (layer "B.Cu") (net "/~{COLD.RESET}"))
 (segment (start 115.085 78.396701) (end 115.085 76.545) (width 0.25) (layer "B.Cu") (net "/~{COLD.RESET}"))
 (segment (start 112.545 78.396701) (end 112.545 76.545) (width 0.25) (layer "B.Cu") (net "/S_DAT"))
 (segment (start 111.7 79.241701) (end 112.545 78.396701) (width 0.25) (layer "B.Cu") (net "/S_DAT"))
 (segment (start 112.545 76.545) (end 111.37 75.37) (width 0.25) (layer "B.Cu") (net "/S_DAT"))
 (segment (start 111.7 114.22) (end 111.7 79.241701) (width 0.25) (layer "B.Cu") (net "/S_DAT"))
 (segment (start 104.925 78.396701) (end 104.925 76.545) (width 0.25) (layer "B.Cu") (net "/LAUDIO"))
 (segment (start 104.2 114.22) (end 104.2 79.121701) (width 0.25) (layer "B.Cu") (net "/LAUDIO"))
 (segment (start 104.925 76.545) (end 103.75 75.37) (width 0.25) (layer "B.Cu") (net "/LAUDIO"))
 (segment (start 104.2 79.121701) (end 104.925 78.396701) (width 0.25) (layer "B.Cu") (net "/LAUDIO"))
 (segment (start 156.7 78.3) (end 157.09 77.91) (width 0.25) (layer "F.Cu") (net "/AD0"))
 (segment (start 156.7 114.22) (end 156.7 78.3) (width 0.25) (layer "F.Cu") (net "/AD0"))
 (segment (start 154.2 78.26) (end 154.55 77.91) (width 0.25) (layer "F.Cu") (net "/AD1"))
 (segment (start 154.2 114.22) (end 154.2 78.26) (width 0.25) (layer "F.Cu") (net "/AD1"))
 (segment (start 151.7 114.22) (end 151.7 78.22) (width 0.25) (layer "F.Cu") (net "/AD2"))
 (segment (start 151.7 78.22) (end 152.01 77.91) (width 0.25) (layer "F.Cu") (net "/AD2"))
 (segment (start 146.7 114.22) (end 146.7 78.14) (width 0.25) (layer "F.Cu") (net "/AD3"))
 (segment (start 146.7 78.14) (end 146.93 77.91) (width 0.25) (layer "F.Cu") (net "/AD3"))
 (segment (start 144.2 114.22) (end 144.2 78.1) (width 0.25) (layer "F.Cu") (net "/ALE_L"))
 (segment (start 144.2 78.1) (end 144.39 77.91) (width 0.25) (layer "F.Cu") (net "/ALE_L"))
 (segment (start 139.2 114.22) (end 139.2 78.02) (width 0.25) (layer "F.Cu") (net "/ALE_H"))
 (segment (start 139.2 78.02) (end 139.31 77.91) (width 0.25) (layer "F.Cu") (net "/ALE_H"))
 (segment (start 136.7 77.98) (end 136.77 77.91) (width 0.25) (layer "F.Cu") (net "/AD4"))
 (segment (start 136.7 114.22) (end 136.7 77.98) (width 0.25) (layer "F.Cu") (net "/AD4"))
 (segment (start 134.2 114.22) (end 134.2 77.94) (width 0.25) (layer "F.Cu") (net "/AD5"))
 (segment (start 134.2 77.94) (end 134.23 77.91) (width 0.25) (layer "F.Cu") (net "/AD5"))
 (segment (start 126.7 114.22) (end 126.7 78) (width 0.25) (layer "F.Cu") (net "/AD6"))
 (segment (start 126.7 78) (end 126.61 77.91) (width 0.25) (layer "F.Cu") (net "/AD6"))
 (segment (start 124.2 78.04) (end 124.07 77.91) (width 0.25) (layer "F.Cu") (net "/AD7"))
 (segment (start 124.2 114.22) (end 124.2 78.04) (width 0.25) (layer "F.Cu") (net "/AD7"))
 (segment (start 119.2 78.12) (end 118.99 77.91) (width 0.25) (layer "F.Cu") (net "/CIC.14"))
 (segment (start 119.2 114.22) (end 119.2 78.12) (width 0.25) (layer "F.Cu") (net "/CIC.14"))
 (segment (start 116.7 114.22) (end 116.7 78.16) (width 0.25) (layer "F.Cu") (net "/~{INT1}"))
 (segment (start 116.7 78.16) (end 116.45 77.91) (width 0.25) (layer "F.Cu") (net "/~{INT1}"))
 (segment (start 114.2 78.2) (end 113.91 77.91) (width 0.25) (layer "F.Cu") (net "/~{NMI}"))
 (segment (start 114.2 114.22) (end 114.2 78.2) (width 0.25) (layer "F.Cu") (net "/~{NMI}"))
 (segment (start 111.7 78.24) (end 111.37 77.91) (width 0.25) (layer "F.Cu") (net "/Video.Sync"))
 (segment (start 111.7 114.22) (end 111.7 78.24) (width 0.25) (layer "F.Cu") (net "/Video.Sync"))
 (segment (start 104.2 78.36) (end 103.75 77.91) (width 0.25) (layer "F.Cu") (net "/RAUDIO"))
 (segment (start 104.2 114.22) (end 104.2 78.36) (width 0.25) (layer "F.Cu") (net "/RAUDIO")))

